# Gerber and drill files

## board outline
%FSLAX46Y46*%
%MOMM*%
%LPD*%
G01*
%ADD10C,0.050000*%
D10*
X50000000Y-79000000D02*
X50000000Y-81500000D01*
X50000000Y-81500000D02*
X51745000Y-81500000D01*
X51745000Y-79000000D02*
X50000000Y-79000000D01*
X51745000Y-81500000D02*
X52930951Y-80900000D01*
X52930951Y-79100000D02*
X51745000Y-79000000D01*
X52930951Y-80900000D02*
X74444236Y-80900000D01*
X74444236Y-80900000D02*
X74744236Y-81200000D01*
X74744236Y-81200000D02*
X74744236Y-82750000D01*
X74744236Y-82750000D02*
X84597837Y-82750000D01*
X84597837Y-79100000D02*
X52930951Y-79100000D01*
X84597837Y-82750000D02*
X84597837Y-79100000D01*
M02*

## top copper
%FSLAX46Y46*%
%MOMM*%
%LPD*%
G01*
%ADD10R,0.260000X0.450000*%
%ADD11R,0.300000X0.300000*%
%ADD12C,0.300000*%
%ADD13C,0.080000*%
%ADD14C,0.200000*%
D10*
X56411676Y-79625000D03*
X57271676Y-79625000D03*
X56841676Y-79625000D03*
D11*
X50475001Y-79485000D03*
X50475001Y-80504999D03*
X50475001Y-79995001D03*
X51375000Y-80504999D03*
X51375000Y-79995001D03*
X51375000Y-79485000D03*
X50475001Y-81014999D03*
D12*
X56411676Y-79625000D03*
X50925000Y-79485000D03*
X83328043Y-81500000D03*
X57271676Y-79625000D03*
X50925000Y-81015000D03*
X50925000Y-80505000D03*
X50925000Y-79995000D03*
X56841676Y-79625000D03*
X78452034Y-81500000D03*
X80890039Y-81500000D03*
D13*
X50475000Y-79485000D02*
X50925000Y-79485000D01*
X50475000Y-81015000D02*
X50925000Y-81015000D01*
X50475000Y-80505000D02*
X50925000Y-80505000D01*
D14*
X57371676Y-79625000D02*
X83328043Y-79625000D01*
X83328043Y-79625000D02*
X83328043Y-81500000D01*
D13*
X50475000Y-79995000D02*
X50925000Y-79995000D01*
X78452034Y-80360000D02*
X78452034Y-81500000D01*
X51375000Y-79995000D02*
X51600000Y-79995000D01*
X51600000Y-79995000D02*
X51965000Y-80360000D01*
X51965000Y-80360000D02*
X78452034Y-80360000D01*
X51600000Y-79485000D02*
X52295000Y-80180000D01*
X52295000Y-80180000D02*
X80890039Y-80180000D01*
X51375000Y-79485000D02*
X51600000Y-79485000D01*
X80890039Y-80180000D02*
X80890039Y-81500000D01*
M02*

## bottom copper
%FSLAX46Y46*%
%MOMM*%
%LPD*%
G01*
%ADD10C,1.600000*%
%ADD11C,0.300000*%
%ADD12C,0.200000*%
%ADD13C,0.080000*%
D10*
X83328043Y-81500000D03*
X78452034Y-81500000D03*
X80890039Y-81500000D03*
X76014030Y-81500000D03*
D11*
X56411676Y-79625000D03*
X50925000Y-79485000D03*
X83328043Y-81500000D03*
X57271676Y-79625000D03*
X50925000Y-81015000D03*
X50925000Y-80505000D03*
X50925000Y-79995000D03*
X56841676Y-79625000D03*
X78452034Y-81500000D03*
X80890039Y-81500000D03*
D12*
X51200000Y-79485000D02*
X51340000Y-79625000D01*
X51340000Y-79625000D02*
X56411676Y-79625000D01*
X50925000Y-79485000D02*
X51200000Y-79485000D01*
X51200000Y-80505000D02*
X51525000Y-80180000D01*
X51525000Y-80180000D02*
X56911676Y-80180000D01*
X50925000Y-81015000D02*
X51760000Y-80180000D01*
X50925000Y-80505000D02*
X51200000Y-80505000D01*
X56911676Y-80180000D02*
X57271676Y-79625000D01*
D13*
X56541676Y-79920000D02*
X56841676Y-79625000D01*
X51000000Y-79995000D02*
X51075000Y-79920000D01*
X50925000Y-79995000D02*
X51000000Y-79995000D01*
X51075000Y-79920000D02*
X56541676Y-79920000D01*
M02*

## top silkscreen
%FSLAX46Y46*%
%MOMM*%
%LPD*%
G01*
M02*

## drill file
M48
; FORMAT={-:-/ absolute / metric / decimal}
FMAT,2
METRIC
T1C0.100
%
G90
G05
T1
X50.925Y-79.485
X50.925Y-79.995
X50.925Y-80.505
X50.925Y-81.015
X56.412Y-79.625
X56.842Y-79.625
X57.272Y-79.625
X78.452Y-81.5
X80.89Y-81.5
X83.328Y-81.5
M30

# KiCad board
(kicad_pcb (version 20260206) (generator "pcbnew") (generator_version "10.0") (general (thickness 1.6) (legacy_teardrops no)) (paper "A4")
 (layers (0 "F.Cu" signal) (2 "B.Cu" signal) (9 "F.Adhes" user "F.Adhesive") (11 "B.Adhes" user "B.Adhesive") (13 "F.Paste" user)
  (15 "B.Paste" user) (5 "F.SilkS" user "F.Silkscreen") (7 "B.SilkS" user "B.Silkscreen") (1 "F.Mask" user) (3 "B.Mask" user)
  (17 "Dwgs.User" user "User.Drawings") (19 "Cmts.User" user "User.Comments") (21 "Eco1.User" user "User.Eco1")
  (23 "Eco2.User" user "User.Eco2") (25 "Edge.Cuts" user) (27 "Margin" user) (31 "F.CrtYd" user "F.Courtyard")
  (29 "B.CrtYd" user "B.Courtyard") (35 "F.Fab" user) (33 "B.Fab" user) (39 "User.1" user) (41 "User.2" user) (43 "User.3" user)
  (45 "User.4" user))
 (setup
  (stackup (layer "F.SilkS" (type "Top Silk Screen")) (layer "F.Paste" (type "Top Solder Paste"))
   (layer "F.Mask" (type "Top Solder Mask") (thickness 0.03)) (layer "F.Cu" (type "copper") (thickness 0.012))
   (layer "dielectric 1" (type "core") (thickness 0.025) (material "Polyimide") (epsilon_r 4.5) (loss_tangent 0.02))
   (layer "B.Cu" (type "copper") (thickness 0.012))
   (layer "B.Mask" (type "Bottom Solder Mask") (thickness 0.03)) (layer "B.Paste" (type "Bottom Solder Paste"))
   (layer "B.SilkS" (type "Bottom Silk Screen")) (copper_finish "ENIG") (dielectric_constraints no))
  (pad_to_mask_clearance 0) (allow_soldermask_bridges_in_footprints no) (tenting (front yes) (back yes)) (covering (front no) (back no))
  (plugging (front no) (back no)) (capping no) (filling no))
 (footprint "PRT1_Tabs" (layer "F.Cu") (at 56.841676 79.625)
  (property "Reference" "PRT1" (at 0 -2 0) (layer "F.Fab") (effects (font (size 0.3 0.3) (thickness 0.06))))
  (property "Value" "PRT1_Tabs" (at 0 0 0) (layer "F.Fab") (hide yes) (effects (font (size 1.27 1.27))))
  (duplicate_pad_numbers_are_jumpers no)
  (pad "1" smd rect (at -0.43 0) (size 0.26 0.45) (layers "F.Cu" "F.Mask") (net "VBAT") (solder_mask_margin 0.05) (thermal_bridge_angle 45))
  (pad "2" smd rect (at 0.43 0) (size 0.26 0.45) (layers "F.Cu" "F.Mask") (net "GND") (solder_mask_margin 0.05) (thermal_bridge_angle 45))
  (pad "3" smd rect (at 0 0) (size 0.26 0.45) (layers "F.Cu" "F.Mask") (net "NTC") (solder_mask_margin 0.05) (thermal_bridge_angle 45)))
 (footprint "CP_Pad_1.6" (layer "F.Cu") (at 83.328043 81.5)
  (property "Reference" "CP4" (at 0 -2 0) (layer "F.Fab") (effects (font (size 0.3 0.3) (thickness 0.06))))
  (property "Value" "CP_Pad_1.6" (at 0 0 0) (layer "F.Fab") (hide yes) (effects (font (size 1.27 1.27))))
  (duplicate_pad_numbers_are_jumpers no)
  (pad "1" smd circle (at 0 0) (size 1.6 1.6) (layers "B.Cu" "B.Mask") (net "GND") (solder_mask_margin 0.1)))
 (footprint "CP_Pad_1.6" (layer "F.Cu") (at 78.452034 81.5)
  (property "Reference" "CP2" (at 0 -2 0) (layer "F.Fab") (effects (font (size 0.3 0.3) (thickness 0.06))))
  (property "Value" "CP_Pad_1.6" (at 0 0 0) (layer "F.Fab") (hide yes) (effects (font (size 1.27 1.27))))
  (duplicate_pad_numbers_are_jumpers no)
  (pad "1" smd circle (at 0 0) (size 1.6 1.6) (layers "B.Cu" "B.Mask") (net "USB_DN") (solder_mask_margin 0.1)))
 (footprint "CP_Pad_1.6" (layer "F.Cu") (at 80.890039 81.5)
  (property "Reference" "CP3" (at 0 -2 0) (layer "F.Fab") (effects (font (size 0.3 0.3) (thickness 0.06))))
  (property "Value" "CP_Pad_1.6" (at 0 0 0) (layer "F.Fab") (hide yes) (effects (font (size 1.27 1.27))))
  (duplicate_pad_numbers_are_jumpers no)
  (pad "1" smd circle (at 0 0) (size 1.6 1.6) (layers "B.Cu" "B.Mask") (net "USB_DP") (solder_mask_margin 0.1)))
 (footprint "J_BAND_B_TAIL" (layer "F.Cu") (at 50.9 80.25)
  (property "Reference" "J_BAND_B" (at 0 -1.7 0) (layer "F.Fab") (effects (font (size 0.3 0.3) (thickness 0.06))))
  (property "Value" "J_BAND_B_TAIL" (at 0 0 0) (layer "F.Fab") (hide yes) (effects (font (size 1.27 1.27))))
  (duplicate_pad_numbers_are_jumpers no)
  (pad "1" smd rect (at -0.424999 -0.765) (size 0.3 0.3) (layers "F.Cu" "F.Mask") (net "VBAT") (solder_mask_margin 0.05)
   (thermal_bridge_angle 45))
  (pad "2" smd rect (at -0.424999 0.254999) (size 0.3 0.3) (layers "F.Cu" "F.Mask") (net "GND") (solder_mask_margin 0.05)
   (thermal_bridge_angle 45))
  (pad "3" smd rect (at -0.424999 -0.254999) (size 0.3 0.3) (layers "F.Cu" "F.Mask") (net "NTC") (solder_mask_margin 0.05)
   (thermal_bridge_angle 45))
  (pad "4" smd rect (at 0.475 0.254999) (size 0.3 0.3) (layers "F.Cu" "F.Mask") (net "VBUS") (solder_mask_margin 0.05)
   (thermal_bridge_angle 45))
  (pad "5" smd rect (at 0.475 -0.254999) (size 0.3 0.3) (layers "F.Cu" "F.Mask") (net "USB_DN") (solder_mask_margin 0.05)
   (thermal_bridge_angle 45))
  (pad "6" smd rect (at 0.475 -0.765) (size 0.3 0.3) (layers "F.Cu" "F.Mask") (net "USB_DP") (solder_mask_margin 0.05)
   (thermal_bridge_angle 45))
  (pad "7" smd rect (at -0.424999 0.764999) (size 0.3 0.3) (layers "F.Cu" "F.Mask") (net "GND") (solder_mask_margin 0.05)
   (thermal_bridge_angle 45)))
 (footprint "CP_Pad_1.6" (layer "F.Cu") (at 76.01403 81.5)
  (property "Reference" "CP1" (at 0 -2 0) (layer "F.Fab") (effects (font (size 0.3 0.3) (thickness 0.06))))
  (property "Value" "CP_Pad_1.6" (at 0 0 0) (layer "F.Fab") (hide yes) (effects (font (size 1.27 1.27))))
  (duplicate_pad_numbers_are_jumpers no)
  (pad "1" smd circle (at 0 0) (size 1.6 1.6) (layers "B.Cu" "B.Mask") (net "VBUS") (solder_mask_margin 0.1)))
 (gr_line (start 50 79) (end 50 81.5) (stroke (width 0.05) (type default)) (layer "Edge.Cuts"))
 (gr_line (start 50 81.5) (end 51.745 81.5) (stroke (width 0.05) (type default)) (layer "Edge.Cuts"))
 (gr_line (start 51.745 79) (end 50 79) (stroke (width 0.05) (type default)) (layer "Edge.Cuts"))
 (gr_line (start 51.745 81.5) (end 52.930951 80.9) (stroke (width 0.05) (type default)) (layer "Edge.Cuts"))
 (gr_line (start 52.930951 79.1) (end 51.745 79) (stroke (width 0.05) (type default)) (layer "Edge.Cuts"))
 (gr_line (start 52.930951 80.9) (end 74.444236 80.9) (stroke (width 0.05) (type default)) (layer "Edge.Cuts"))
 (gr_line (start 74.444236 80.9) (end 74.744236 81.2) (stroke (width 0.05) (type default)) (layer "Edge.Cuts"))
 (gr_line (start 74.744236 81.2) (end 74.744236 82.75) (stroke (width 0.05) (type default)) (layer "Edge.Cuts"))
 (gr_line (start 74.744236 82.75) (end 84.597837 82.75) (stroke (width 0.05) (type default)) (layer "Edge.Cuts"))
 (gr_line (start 84.597837 79.1) (end 52.930951 79.1) (stroke (width 0.05) (type default)) (layer "Edge.Cuts"))
 (gr_line (start 84.597837 82.75) (end 84.597837 79.1) (stroke (width 0.05) (type default)) (layer "Edge.Cuts"))
 (segment (start 50.475 79.485) (end 50.925 79.485) (width 0.08) (layer "F.Cu") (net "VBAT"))
 (via (at 56.411676 79.625) (size 0.3) (drill 0.1) (layers "F.Cu" "B.Cu") (tenting (front yes) (back yes)) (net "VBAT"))
 (via (at 50.925 79.485) (size 0.3) (drill 0.1) (layers "F.Cu" "B.Cu") (tenting (front yes) (back yes)) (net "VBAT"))
 (segment (start 51.2 79.485) (end 51.34 79.625) (width 0.2) (layer "B.Cu") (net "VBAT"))
 (segment (start 51.34 79.625) (end 56.411676 79.625) (width 0.2) (layer "B.Cu") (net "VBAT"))
 (segment (start 50.925 79.485) (end 51.2 79.485) (width 0.2) (layer "B.Cu") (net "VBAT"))
 (segment (start 50.475 81.015) (end 50.925 81.015) (width 0.08) (layer "F.Cu") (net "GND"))
 (segment (start 50.475 80.505) (end 50.925 80.505) (width 0.08) (layer "F.Cu") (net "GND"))
 (segment (start 57.371676 79.625) (end 83.328043 79.625) (width 0.2) (layer "F.Cu") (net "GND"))
 (segment (start 83.328043 79.625) (end 83.328043 81.5) (width 0.2) (layer "F.Cu") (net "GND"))
 (via (at 83.328043 81.5) (size 0.3) (drill 0.1) (layers "F.Cu" "B.Cu") (tenting (front yes) (back yes)) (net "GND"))
 (via (at 57.271676 79.625) (size 0.3) (drill 0.1) (layers "F.Cu" "B.Cu") (tenting (front yes) (back yes)) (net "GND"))
 (via (at 50.925 81.015) (size 0.3) (drill 0.1) (layers "F.Cu" "B.Cu") (tenting (front yes) (back yes)) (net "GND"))
 (via (at 50.925 80.505) (size 0.3) (drill 0.1) (layers "F.Cu" "B.Cu") (tenting (front yes) (back yes)) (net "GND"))
 (segment (start 51.2 80.505) (end 51.525 80.18) (width 0.2) (layer "B.Cu") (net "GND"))
 (segment (start 51.525 80.18) (end 56.911676 80.18) (width 0.2) (layer "B.Cu") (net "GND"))
 (segment (start 50.925 81.015) (end 51.76 80.18) (width 0.2) (layer "B.Cu") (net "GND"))
 (segment (start 50.925 80.505) (end 51.2 80.505) (width 0.2) (layer "B.Cu") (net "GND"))
 (segment (start 56.911676 80.18) (end 57.271676 79.625) (width 0.2) (layer "B.Cu") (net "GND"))
 (segment (start 50.475 79.995) (end 50.925 79.995) (width 0.08) (layer "F.Cu") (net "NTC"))
 (via (at 50.925 79.995) (size 0.3) (drill 0.1) (layers "F.Cu" "B.Cu") (tenting (front yes) (back yes)) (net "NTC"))
 (via (at 56.841676 79.625) (size 0.3) (drill 0.1) (layers "F.Cu" "B.Cu") (tenting (front yes) (back yes)) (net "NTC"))
 (segment (start 56.541676 79.92) (end 56.841676 79.625) (width 0.08) (layer "B.Cu") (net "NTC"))
 (segment (start 51 79.995) (end 51.075 79.92) (width 0.08) (layer "B.Cu") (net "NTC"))
 (segment (start 50.925 79.995) (end 51 79.995) (width 0.08) (layer "B.Cu") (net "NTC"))
 (segment (start 51.075 79.92) (end 56.541676 79.92) (width 0.08) (layer "B.Cu") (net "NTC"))
 (segment (start 78.452034 80.36) (end 78.452034 81.5) (width 0.08) (layer "F.Cu") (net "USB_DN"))
 (segment (start 51.375 79.995) (end 51.6 79.995) (width 0.08) (layer "F.Cu") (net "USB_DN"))
 (segment (start 51.6 79.995) (end 51.965 80.36) (width 0.08) (layer "F.Cu") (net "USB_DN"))
 (segment (start 51.965 80.36) (end 78.452034 80.36) (width 0.08) (layer "F.Cu") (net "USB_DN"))
 (via (at 78.452034 81.5) (size 0.3) (drill 0.1) (layers "F.Cu" "B.Cu") (tenting (front yes) (back yes)) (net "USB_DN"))
 (segment (start 51.6 79.485) (end 52.295 80.18) (width 0.08) (layer "F.Cu") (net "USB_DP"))
 (segment (start 52.295 80.18) (end 80.890039 80.18) (width 0.08) (layer "F.Cu") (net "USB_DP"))
 (segment (start 51.375 79.485) (end 51.6 79.485) (width 0.08) (layer "F.Cu") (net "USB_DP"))
 (segment (start 80.890039 80.18) (end 80.890039 81.5) (width 0.08) (layer "F.Cu") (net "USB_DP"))
 (via (at 80.890039 81.5) (size 0.3) (drill 0.1) (layers "F.Cu" "B.Cu") (tenting (front yes) (back yes)) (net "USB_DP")))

